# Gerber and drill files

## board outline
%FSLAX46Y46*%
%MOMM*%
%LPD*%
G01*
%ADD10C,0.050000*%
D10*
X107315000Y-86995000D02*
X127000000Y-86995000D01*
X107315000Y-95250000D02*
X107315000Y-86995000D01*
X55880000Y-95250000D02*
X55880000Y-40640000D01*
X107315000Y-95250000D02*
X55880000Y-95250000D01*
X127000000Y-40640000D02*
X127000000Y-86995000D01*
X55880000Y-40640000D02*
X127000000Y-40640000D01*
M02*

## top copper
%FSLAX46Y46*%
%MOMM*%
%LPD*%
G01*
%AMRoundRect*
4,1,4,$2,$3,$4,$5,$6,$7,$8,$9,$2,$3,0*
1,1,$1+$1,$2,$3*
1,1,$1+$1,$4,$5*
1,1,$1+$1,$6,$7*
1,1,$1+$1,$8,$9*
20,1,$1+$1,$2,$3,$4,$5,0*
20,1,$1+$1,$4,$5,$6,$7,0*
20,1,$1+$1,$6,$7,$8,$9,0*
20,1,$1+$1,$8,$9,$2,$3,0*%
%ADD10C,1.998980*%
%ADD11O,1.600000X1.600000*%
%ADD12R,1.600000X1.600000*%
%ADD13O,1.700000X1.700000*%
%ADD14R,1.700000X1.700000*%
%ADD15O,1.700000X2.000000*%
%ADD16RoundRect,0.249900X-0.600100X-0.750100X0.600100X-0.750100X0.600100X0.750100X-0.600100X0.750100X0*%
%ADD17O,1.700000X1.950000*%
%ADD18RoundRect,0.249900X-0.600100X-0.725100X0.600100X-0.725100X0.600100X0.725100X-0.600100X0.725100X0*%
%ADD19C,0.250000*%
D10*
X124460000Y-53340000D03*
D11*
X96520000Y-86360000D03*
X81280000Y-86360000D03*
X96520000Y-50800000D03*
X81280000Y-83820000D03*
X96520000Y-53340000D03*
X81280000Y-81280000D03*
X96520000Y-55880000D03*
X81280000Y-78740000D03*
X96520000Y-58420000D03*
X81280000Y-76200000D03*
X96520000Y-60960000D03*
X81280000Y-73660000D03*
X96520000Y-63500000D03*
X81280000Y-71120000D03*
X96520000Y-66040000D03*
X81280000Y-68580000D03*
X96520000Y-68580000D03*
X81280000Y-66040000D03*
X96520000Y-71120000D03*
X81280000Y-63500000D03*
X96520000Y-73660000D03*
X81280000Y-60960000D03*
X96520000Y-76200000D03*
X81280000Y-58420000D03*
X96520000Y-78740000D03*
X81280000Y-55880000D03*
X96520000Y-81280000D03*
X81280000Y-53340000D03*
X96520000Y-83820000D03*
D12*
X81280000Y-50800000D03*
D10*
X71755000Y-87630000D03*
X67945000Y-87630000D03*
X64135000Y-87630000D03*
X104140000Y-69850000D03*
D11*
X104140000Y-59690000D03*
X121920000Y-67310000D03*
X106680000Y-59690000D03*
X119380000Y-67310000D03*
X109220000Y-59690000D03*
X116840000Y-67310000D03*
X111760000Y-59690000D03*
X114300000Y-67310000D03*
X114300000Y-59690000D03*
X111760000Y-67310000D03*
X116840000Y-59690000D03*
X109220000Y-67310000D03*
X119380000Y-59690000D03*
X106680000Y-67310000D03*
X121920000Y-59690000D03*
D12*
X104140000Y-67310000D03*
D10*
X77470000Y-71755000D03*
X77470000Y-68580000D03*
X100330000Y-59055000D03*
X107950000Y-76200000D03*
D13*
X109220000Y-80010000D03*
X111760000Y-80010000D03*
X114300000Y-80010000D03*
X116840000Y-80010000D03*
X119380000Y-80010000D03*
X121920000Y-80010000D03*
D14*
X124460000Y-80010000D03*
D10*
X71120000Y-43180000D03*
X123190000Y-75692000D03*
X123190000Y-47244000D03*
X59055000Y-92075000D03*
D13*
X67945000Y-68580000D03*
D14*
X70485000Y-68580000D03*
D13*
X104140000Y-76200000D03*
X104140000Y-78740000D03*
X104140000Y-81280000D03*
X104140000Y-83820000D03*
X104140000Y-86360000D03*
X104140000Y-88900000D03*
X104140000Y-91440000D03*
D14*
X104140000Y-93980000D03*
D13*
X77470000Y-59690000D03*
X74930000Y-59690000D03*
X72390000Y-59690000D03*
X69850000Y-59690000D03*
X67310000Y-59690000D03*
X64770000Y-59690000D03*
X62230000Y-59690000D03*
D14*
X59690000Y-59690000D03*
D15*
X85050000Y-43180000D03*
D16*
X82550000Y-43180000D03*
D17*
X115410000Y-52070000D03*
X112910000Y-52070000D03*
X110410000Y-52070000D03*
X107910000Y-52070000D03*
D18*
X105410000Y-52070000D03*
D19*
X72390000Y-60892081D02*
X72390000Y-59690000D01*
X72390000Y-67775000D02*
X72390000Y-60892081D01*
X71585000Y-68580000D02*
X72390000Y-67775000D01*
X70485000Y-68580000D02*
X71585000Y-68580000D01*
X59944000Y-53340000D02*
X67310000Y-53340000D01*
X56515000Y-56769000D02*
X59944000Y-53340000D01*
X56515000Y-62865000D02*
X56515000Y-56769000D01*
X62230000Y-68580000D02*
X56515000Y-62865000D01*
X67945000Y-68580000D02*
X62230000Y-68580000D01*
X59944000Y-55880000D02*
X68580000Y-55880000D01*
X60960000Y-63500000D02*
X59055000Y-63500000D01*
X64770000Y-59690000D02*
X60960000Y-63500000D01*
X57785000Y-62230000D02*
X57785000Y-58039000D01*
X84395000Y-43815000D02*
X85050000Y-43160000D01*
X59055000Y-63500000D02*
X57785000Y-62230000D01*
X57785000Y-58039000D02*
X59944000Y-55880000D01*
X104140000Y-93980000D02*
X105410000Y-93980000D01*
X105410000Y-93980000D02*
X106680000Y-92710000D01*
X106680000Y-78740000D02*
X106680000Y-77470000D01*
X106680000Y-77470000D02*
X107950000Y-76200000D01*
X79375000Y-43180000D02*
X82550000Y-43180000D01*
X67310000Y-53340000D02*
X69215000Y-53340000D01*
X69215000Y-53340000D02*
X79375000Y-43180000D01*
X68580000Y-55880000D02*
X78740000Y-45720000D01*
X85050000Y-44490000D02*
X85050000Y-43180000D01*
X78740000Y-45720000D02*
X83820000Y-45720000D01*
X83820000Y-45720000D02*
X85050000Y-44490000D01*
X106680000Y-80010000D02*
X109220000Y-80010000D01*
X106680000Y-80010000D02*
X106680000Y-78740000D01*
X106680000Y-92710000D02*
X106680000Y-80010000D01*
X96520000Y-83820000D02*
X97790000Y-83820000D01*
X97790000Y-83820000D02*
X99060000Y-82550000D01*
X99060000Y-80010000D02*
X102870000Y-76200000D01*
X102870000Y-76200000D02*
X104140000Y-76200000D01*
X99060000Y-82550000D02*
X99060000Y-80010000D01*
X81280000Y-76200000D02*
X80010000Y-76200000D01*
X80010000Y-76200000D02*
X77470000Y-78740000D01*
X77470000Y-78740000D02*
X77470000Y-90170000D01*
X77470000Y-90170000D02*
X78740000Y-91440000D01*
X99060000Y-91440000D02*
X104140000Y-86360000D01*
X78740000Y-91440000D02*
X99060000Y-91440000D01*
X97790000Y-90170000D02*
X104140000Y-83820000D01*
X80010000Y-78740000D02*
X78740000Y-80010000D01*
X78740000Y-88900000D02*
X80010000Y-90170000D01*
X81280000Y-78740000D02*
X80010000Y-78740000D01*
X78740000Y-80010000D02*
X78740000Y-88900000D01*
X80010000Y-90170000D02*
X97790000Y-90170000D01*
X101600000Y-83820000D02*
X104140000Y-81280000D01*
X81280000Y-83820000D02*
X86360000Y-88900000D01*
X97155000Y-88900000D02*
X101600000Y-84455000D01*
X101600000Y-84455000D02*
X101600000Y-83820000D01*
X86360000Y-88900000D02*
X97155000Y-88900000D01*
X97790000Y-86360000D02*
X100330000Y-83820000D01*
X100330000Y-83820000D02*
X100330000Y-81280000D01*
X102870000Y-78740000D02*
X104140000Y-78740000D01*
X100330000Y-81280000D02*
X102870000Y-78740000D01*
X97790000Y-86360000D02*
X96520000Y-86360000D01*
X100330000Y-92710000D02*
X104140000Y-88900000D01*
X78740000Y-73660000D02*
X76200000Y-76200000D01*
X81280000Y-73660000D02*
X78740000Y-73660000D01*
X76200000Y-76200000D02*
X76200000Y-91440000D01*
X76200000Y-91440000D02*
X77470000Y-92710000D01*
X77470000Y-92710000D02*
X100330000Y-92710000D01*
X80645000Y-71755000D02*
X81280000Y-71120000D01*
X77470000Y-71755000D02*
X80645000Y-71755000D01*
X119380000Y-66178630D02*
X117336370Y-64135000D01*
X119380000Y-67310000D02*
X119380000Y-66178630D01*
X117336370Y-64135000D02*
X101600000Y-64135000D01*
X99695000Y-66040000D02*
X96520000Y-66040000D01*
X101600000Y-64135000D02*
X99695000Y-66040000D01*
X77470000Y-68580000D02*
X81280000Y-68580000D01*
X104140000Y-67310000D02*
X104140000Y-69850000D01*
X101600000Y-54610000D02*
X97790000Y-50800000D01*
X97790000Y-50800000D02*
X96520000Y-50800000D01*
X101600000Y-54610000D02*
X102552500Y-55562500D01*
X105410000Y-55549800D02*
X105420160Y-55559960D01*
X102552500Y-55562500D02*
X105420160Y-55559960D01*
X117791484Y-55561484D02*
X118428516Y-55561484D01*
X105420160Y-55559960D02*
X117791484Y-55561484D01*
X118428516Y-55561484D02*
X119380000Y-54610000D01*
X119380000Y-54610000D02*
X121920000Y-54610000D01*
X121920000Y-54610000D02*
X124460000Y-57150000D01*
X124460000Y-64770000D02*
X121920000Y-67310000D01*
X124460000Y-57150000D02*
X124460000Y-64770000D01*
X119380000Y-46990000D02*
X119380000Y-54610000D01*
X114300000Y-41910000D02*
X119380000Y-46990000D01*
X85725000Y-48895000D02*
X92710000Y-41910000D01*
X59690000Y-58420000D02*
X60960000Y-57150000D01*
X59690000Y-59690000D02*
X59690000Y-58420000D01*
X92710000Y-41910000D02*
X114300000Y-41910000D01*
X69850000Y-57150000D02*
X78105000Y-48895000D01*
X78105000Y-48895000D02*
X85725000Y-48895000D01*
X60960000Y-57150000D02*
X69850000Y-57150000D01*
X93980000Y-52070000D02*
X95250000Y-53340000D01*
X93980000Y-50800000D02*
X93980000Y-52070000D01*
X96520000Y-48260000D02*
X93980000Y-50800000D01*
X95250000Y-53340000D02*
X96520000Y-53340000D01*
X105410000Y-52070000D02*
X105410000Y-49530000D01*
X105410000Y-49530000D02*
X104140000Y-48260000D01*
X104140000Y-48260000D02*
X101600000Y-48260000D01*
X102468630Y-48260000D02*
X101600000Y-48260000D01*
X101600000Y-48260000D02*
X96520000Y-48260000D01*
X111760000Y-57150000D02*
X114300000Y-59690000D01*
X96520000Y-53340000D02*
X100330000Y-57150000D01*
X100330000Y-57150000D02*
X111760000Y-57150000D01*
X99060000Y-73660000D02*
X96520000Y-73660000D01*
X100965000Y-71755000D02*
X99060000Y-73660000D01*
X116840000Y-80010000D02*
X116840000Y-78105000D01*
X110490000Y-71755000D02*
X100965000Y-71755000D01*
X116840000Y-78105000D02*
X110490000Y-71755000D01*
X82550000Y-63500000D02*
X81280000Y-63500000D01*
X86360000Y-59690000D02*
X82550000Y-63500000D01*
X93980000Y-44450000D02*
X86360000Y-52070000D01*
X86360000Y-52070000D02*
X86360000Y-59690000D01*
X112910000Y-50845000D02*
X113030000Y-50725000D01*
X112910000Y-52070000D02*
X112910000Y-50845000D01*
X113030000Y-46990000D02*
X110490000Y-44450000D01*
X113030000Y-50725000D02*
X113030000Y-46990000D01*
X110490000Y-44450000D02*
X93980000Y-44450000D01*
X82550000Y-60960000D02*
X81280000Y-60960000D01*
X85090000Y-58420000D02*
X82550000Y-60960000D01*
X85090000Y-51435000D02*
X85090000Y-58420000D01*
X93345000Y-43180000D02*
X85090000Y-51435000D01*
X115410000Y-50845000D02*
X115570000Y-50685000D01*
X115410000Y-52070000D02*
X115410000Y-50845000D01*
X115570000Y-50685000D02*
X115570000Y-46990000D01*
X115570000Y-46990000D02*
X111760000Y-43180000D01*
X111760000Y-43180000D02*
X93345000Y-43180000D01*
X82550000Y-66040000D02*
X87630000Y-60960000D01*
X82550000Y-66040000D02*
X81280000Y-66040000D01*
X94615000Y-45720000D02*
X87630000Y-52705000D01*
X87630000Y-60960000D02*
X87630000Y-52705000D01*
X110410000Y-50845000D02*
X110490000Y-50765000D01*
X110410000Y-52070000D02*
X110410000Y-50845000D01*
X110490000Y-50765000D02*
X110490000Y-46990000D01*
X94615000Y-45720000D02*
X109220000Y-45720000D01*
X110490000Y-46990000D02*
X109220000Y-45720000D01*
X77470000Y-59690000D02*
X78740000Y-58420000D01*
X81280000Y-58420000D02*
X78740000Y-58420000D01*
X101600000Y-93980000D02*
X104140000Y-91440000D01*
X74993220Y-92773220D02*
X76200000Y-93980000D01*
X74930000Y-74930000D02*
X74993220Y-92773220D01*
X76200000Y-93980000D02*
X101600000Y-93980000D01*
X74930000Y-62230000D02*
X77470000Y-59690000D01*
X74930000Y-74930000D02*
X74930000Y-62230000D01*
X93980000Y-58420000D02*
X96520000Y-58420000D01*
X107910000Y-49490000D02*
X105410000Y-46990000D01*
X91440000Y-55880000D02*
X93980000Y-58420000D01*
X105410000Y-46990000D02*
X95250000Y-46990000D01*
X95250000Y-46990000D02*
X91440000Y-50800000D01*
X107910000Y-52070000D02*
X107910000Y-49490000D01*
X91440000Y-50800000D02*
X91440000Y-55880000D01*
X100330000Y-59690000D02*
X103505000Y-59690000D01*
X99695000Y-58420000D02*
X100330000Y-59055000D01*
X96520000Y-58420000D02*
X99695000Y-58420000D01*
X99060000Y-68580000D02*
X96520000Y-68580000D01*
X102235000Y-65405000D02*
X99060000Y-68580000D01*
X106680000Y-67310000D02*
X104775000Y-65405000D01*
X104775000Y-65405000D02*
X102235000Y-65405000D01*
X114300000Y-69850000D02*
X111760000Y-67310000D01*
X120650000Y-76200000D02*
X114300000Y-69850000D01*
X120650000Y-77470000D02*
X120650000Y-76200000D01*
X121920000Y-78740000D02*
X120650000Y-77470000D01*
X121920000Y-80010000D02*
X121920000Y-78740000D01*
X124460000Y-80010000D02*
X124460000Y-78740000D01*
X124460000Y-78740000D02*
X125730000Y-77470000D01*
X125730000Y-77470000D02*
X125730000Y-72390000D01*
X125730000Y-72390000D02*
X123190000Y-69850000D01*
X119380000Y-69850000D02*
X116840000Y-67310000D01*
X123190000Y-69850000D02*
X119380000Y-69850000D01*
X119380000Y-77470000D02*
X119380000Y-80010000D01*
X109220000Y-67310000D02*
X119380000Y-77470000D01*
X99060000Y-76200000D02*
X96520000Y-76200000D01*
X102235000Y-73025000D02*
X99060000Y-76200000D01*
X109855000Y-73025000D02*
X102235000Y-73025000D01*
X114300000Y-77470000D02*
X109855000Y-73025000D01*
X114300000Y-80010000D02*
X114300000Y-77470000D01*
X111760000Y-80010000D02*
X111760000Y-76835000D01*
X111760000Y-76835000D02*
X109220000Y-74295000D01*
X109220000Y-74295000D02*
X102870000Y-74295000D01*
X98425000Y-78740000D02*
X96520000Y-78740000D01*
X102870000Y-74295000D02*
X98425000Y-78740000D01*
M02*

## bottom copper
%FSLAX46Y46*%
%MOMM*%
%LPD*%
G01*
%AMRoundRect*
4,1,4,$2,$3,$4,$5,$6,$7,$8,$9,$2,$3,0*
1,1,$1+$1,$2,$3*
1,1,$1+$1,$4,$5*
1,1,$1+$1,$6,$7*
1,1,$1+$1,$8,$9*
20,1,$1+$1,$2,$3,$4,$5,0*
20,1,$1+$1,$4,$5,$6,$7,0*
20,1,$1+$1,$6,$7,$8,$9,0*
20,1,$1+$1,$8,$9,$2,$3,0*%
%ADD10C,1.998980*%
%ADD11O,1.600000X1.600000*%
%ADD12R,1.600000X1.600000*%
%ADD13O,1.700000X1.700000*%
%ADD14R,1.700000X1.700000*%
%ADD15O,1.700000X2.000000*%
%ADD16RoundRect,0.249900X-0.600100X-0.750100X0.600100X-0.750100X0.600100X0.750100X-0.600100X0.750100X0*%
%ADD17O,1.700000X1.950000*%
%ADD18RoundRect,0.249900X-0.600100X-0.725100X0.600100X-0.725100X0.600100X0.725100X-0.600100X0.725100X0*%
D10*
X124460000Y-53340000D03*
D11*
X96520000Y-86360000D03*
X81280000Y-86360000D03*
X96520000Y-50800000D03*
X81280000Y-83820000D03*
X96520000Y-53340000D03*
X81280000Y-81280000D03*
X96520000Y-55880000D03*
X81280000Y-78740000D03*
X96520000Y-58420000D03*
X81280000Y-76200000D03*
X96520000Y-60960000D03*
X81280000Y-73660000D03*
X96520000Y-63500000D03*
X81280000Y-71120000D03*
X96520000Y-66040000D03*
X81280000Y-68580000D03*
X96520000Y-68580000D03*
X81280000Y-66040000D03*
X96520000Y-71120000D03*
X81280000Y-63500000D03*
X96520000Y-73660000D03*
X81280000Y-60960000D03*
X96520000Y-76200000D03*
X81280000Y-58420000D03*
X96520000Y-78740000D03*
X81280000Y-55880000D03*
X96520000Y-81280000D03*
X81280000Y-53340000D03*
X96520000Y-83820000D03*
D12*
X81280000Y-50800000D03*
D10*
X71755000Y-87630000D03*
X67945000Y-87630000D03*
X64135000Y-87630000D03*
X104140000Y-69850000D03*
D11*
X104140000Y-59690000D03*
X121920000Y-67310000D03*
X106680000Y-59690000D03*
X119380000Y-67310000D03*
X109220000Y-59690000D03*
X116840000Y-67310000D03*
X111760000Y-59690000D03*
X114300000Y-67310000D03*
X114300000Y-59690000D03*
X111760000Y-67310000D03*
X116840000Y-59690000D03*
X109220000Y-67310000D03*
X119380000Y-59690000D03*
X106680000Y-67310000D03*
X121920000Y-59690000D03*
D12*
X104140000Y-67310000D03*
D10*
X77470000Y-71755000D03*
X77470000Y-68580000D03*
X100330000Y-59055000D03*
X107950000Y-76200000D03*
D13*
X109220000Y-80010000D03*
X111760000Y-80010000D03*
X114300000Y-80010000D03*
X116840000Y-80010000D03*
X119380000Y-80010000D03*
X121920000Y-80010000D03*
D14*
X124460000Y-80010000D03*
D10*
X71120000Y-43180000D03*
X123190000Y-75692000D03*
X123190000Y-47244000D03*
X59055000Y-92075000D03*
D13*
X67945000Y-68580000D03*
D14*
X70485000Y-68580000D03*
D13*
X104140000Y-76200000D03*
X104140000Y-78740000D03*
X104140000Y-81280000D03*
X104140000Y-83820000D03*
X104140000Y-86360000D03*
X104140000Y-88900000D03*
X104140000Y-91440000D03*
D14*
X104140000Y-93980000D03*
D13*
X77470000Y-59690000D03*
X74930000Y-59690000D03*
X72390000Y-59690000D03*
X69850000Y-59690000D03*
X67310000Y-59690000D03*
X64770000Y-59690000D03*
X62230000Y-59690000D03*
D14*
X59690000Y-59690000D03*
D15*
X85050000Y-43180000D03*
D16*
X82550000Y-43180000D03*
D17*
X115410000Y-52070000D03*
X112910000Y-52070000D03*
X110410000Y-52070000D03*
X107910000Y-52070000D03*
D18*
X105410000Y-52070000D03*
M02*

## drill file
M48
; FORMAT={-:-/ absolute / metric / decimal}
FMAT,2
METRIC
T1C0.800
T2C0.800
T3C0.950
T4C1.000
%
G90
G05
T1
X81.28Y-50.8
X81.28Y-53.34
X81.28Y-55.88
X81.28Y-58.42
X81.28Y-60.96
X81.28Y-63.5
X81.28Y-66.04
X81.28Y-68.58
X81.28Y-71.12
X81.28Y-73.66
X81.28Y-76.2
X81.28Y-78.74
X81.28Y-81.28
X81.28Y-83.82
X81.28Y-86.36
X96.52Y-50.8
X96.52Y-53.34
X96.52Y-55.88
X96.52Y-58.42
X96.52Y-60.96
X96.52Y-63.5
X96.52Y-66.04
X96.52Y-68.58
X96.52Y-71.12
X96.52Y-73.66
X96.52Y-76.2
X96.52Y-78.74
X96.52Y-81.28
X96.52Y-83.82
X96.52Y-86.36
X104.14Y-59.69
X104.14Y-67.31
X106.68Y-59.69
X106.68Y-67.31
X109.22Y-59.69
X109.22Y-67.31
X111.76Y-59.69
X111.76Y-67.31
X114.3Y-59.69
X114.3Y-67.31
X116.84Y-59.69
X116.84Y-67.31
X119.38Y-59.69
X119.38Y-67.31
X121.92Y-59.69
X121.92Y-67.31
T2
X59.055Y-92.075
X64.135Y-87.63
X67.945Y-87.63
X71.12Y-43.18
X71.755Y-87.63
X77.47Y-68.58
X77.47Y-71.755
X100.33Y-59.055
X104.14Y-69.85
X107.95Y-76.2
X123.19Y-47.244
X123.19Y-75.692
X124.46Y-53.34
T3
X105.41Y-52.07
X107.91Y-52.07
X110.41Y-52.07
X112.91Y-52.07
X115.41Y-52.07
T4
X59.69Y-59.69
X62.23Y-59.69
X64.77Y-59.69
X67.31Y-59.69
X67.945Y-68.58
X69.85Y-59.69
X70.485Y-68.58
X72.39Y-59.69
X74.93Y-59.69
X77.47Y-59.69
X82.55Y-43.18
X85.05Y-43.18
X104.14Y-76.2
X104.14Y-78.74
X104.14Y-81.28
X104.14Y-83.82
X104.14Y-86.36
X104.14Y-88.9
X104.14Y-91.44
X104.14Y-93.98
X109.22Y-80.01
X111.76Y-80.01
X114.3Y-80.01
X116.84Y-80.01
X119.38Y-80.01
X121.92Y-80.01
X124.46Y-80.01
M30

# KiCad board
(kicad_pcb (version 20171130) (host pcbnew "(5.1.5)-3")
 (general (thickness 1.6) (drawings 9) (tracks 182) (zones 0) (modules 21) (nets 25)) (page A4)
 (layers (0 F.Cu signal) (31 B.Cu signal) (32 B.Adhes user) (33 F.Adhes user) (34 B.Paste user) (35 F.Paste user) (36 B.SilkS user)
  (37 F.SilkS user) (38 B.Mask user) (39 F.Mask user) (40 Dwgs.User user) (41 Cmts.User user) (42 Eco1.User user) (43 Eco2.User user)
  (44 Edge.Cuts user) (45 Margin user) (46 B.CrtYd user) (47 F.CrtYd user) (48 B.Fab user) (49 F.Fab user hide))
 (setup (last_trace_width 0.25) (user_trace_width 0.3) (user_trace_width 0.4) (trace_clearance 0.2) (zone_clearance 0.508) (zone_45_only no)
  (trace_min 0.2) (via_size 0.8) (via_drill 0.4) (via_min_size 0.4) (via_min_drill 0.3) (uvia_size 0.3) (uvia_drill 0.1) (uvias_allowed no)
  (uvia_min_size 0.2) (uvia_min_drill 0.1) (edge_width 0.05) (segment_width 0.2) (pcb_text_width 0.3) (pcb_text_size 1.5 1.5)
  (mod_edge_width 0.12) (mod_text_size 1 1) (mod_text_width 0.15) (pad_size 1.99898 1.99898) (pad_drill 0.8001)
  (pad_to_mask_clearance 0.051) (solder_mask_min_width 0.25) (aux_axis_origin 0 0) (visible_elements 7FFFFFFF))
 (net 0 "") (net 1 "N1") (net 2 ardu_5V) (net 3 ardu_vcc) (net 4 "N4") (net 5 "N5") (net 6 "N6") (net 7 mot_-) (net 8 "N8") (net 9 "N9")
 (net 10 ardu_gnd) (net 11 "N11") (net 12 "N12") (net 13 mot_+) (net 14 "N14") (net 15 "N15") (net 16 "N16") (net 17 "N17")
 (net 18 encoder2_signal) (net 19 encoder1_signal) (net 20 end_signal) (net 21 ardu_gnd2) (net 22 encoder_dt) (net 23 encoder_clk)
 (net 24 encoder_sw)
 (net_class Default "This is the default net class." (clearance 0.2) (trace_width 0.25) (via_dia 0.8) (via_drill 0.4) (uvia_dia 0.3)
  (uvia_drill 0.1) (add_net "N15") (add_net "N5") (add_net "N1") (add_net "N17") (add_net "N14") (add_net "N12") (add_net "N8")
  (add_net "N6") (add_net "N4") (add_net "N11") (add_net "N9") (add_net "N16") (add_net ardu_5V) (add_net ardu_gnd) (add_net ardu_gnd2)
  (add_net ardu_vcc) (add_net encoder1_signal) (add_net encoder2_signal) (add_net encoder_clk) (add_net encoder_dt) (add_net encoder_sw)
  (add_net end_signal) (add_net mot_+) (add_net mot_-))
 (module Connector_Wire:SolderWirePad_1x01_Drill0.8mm (layer F.Cu) (at 124.46 53.34)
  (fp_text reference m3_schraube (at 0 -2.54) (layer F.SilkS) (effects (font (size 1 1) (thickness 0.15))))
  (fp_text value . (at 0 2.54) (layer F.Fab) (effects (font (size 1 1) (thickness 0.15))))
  (pad 1 thru_hole circle (at 0 0) (size 1.99898 1.99898) (drill 0.8001) (layers *.Cu *.Mask)))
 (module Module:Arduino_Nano (layer F.Cu) (at 81.28 50.8)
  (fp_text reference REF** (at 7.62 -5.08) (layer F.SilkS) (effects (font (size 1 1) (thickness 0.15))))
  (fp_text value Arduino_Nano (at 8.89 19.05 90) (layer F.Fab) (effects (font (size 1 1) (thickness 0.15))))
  (pad 16 thru_hole oval (at 15.24 35.56) (size 1.6 1.6) (drill 0.8) (layers *.Cu *.Mask))
  (pad 15 thru_hole oval (at 0 35.56) (size 1.6 1.6) (drill 0.8) (layers *.Cu *.Mask))
  (pad 30 thru_hole oval (at 15.24 0) (size 1.6 1.6) (drill 0.8) (layers *.Cu *.Mask))
  (pad 14 thru_hole oval (at 0 33.02) (size 1.6 1.6) (drill 0.8) (layers *.Cu *.Mask))
  (pad 29 thru_hole oval (at 15.24 2.54) (size 1.6 1.6) (drill 0.8) (layers *.Cu *.Mask))
  (pad 13 thru_hole oval (at 0 30.48) (size 1.6 1.6) (drill 0.8) (layers *.Cu *.Mask))
  (pad 28 thru_hole oval (at 15.24 5.08) (size 1.6 1.6) (drill 0.8) (layers *.Cu *.Mask))
  (pad 12 thru_hole oval (at 0 27.94) (size 1.6 1.6) (drill 0.8) (layers *.Cu *.Mask))
  (pad 27 thru_hole oval (at 15.24 7.62) (size 1.6 1.6) (drill 0.8) (layers *.Cu *.Mask))
  (pad 11 thru_hole oval (at 0 25.4) (size 1.6 1.6) (drill 0.8) (layers *.Cu *.Mask))
  (pad 26 thru_hole oval (at 15.24 10.16) (size 1.6 1.6) (drill 0.8) (layers *.Cu *.Mask))
  (pad 10 thru_hole oval (at 0 22.86) (size 1.6 1.6) (drill 0.8) (layers *.Cu *.Mask))
  (pad 25 thru_hole oval (at 15.24 12.7) (size 1.6 1.6) (drill 0.8) (layers *.Cu *.Mask))
  (pad 9 thru_hole oval (at 0 20.32) (size 1.6 1.6) (drill 0.8) (layers *.Cu *.Mask))
  (pad 24 thru_hole oval (at 15.24 15.24) (size 1.6 1.6) (drill 0.8) (layers *.Cu *.Mask))
  (pad 8 thru_hole oval (at 0 17.78) (size 1.6 1.6) (drill 0.8) (layers *.Cu *.Mask))
  (pad 23 thru_hole oval (at 15.24 17.78) (size 1.6 1.6) (drill 0.8) (layers *.Cu *.Mask))
  (pad 7 thru_hole oval (at 0 15.24) (size 1.6 1.6) (drill 0.8) (layers *.Cu *.Mask))
  (pad 22 thru_hole oval (at 15.24 20.32) (size 1.6 1.6) (drill 0.8) (layers *.Cu *.Mask))
  (pad 6 thru_hole oval (at 0 12.7) (size 1.6 1.6) (drill 0.8) (layers *.Cu *.Mask))
  (pad 21 thru_hole oval (at 15.24 22.86) (size 1.6 1.6) (drill 0.8) (layers *.Cu *.Mask))
  (pad 5 thru_hole oval (at 0 10.16) (size 1.6 1.6) (drill 0.8) (layers *.Cu *.Mask))
  (pad 20 thru_hole oval (at 15.24 25.4) (size 1.6 1.6) (drill 0.8) (layers *.Cu *.Mask))
  (pad 4 thru_hole oval (at 0 7.62) (size 1.6 1.6) (drill 0.8) (layers *.Cu *.Mask))
  (pad 19 thru_hole oval (at 15.24 27.94) (size 1.6 1.6) (drill 0.8) (layers *.Cu *.Mask))
  (pad 3 thru_hole oval (at 0 5.08) (size 1.6 1.6) (drill 0.8) (layers *.Cu *.Mask))
  (pad 18 thru_hole oval (at 15.24 30.48) (size 1.6 1.6) (drill 0.8) (layers *.Cu *.Mask))
  (pad 2 thru_hole oval (at 0 2.54) (size 1.6 1.6) (drill 0.8) (layers *.Cu *.Mask))
  (pad 17 thru_hole oval (at 15.24 33.02) (size 1.6 1.6) (drill 0.8) (layers *.Cu *.Mask))
  (pad 1 thru_hole rect (at 0 0) (size 1.6 1.6) (drill 0.8) (layers *.Cu *.Mask)))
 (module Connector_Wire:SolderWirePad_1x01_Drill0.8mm (layer F.Cu) (at 71.755 87.63)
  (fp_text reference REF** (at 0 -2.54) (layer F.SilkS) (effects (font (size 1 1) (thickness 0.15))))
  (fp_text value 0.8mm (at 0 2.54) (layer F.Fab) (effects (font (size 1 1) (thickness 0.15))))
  (pad 1 thru_hole circle (at 0 0) (size 1.99898 1.99898) (drill 0.8001) (layers *.Cu *.Mask)))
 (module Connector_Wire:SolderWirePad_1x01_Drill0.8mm (layer F.Cu) (at 67.945 87.63)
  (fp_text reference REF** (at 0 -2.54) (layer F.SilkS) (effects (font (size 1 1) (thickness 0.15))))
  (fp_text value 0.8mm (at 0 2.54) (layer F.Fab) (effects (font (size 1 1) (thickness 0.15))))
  (pad 1 thru_hole circle (at 0 0) (size 1.99898 1.99898) (drill 0.8001) (layers *.Cu *.Mask)))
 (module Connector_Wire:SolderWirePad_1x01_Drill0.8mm (layer F.Cu) (at 64.135 87.63)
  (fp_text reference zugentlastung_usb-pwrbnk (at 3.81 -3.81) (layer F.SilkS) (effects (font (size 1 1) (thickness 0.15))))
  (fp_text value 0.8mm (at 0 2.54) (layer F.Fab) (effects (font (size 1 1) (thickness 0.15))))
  (pad 1 thru_hole circle (at 0 0) (size 1.99898 1.99898) (drill 0.8001) (layers *.Cu *.Mask)))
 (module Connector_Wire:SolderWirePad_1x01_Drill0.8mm (layer F.Cu) (at 104.14 69.85)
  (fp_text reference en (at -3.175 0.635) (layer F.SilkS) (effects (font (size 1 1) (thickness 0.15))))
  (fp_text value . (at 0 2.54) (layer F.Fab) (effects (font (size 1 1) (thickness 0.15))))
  (pad 1 thru_hole circle (at 0 0) (size 1.99898 1.99898) (drill 0.8001) (layers *.Cu *.Mask) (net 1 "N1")))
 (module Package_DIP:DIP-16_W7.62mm (layer F.Cu) (at 104.14 67.31 90)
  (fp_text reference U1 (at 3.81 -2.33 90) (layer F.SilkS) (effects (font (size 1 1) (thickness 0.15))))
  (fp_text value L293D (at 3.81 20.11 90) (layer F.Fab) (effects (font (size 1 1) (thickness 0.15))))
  (pad 16 thru_hole oval (at 7.62 0 90) (size 1.6 1.6) (drill 0.8) (layers *.Cu *.Mask) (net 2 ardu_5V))
  (pad 8 thru_hole oval (at 0 17.78 90) (size 1.6 1.6) (drill 0.8) (layers *.Cu *.Mask) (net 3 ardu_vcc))
  (pad 15 thru_hole oval (at 7.62 2.54 90) (size 1.6 1.6) (drill 0.8) (layers *.Cu *.Mask) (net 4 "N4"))
  (pad 7 thru_hole oval (at 0 15.24 90) (size 1.6 1.6) (drill 0.8) (layers *.Cu *.Mask) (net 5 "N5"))
  (pad 14 thru_hole oval (at 7.62 5.08 90) (size 1.6 1.6) (drill 0.8) (layers *.Cu *.Mask) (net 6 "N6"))
  (pad 6 thru_hole oval (at 0 12.7 90) (size 1.6 1.6) (drill 0.8) (layers *.Cu *.Mask) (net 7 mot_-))
  (pad 13 thru_hole oval (at 7.62 7.62 90) (size 1.6 1.6) (drill 0.8) (layers *.Cu *.Mask) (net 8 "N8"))
  (pad 5 thru_hole oval (at 0 10.16 90) (size 1.6 1.6) (drill 0.8) (layers *.Cu *.Mask) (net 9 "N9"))
  (pad 12 thru_hole oval (at 7.62 10.16 90) (size 1.6 1.6) (drill 0.8) (layers *.Cu *.Mask) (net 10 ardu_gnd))
  (pad 4 thru_hole oval (at 0 7.62 90) (size 1.6 1.6) (drill 0.8) (layers *.Cu *.Mask) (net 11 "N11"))
  (pad 11 thru_hole oval (at 7.62 12.7 90) (size 1.6 1.6) (drill 0.8) (layers *.Cu *.Mask) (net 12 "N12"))
  (pad 3 thru_hole oval (at 0 5.08 90) (size 1.6 1.6) (drill 0.8) (layers *.Cu *.Mask) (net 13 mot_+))
  (pad 10 thru_hole oval (at 7.62 15.24 90) (size 1.6 1.6) (drill 0.8) (layers *.Cu *.Mask) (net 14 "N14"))
  (pad 2 thru_hole oval (at 0 2.54 90) (size 1.6 1.6) (drill 0.8) (layers *.Cu *.Mask) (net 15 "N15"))
  (pad 9 thru_hole oval (at 7.62 17.78 90) (size 1.6 1.6) (drill 0.8) (layers *.Cu *.Mask) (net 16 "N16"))
  (pad 1 thru_hole rect (at 0 0 90) (size 1.6 1.6) (drill 0.8) (layers *.Cu *.Mask) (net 1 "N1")))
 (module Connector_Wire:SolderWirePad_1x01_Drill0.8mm (layer F.Cu) (at 77.47 71.755)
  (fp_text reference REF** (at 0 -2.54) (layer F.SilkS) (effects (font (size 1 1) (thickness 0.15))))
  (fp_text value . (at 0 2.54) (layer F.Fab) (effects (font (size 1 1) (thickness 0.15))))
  (pad 1 thru_hole circle (at 0 0) (size 1.99898 1.99898) (drill 0.8001) (layers *.Cu *.Mask) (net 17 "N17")))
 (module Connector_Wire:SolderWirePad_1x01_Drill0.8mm (layer F.Cu) (at 77.47 68.58)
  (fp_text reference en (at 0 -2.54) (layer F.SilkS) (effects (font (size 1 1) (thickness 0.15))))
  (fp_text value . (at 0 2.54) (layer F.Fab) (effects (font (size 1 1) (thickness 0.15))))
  (pad 1 thru_hole circle (at 0 0) (size 1.99898 1.99898) (drill 0.8001) (layers *.Cu *.Mask) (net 1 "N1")))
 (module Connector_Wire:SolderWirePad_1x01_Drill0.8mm (layer F.Cu) (at 100.33 59.055)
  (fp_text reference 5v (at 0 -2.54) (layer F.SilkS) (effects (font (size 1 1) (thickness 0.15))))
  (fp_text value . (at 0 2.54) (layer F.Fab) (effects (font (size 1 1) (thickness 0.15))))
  (pad 1 thru_hole circle (at 0 0) (size 1.99898 1.99898) (drill 0.8001) (layers *.Cu *.Mask) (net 2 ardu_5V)))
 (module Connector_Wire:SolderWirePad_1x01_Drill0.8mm (layer F.Cu) (at 107.95 76.2)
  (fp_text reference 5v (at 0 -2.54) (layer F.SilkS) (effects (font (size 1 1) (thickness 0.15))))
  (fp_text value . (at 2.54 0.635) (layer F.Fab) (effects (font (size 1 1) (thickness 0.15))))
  (pad 1 thru_hole circle (at 0 0) (size 1.99898 1.99898) (drill 0.8001) (layers *.Cu *.Mask)))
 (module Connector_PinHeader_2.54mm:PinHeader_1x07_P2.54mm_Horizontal (layer F.Cu) (at 124.46 80.01 270)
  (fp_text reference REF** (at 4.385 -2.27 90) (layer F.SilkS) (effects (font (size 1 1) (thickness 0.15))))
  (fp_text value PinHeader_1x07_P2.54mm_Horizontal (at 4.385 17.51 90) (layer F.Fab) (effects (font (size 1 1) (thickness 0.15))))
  (pad 7 thru_hole oval (at 0 15.24 270) (size 1.7 1.7) (drill 1) (layers *.Cu *.Mask))
  (pad 6 thru_hole oval (at 0 12.7 270) (size 1.7 1.7) (drill 1) (layers *.Cu *.Mask) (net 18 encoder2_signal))
  (pad 5 thru_hole oval (at 0 10.16 270) (size 1.7 1.7) (drill 1) (layers *.Cu *.Mask) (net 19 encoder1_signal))
  (pad 4 thru_hole oval (at 0 7.62 270) (size 1.7 1.7) (drill 1) (layers *.Cu *.Mask) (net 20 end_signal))
  (pad 3 thru_hole oval (at 0 5.08 270) (size 1.7 1.7) (drill 1) (layers *.Cu *.Mask) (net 13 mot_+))
  (pad 2 thru_hole oval (at 0 2.54 270) (size 1.7 1.7) (drill 1) (layers *.Cu *.Mask) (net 11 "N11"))
  (pad 1 thru_hole rect (at 0 0 270) (size 1.7 1.7) (drill 1) (layers *.Cu *.Mask) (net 7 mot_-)))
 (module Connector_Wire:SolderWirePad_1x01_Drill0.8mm (layer F.Cu) (at 71.12 43.18)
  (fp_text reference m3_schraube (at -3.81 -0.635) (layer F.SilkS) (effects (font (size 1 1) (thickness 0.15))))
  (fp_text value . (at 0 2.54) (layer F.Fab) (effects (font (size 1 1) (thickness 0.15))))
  (pad 1 thru_hole circle (at 0 0) (size 1.99898 1.99898) (drill 0.8001) (layers *.Cu *.Mask)))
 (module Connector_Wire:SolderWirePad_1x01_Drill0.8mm (layer F.Cu) (at 123.19 75.692)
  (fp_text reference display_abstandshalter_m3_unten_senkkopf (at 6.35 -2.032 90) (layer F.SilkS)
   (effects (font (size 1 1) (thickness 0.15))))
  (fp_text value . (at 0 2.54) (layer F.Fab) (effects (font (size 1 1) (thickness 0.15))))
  (pad 1 thru_hole circle (at 0 0) (size 1.99898 1.99898) (drill 0.8001) (layers *.Cu *.Mask)))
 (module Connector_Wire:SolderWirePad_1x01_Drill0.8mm (layer F.Cu) (at 123.19 47.244)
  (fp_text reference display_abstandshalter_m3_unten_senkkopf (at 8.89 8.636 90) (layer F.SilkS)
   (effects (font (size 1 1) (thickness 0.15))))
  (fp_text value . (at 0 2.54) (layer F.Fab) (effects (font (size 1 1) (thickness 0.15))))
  (pad 1 thru_hole circle (at 0 0) (size 1.99898 1.99898) (drill 0.8001) (layers *.Cu *.Mask)))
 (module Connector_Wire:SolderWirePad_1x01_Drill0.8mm (layer F.Cu) (at 59.055 92.075)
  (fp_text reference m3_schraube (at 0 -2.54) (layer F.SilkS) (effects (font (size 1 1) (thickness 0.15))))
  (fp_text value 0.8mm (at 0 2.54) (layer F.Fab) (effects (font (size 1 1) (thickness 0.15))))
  (pad 1 thru_hole circle (at 0 0) (size 1.99898 1.99898) (drill 0.8001) (layers *.Cu *.Mask)))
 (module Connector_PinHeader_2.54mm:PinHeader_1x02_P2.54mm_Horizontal (layer F.Cu) (at 70.485 68.58 270)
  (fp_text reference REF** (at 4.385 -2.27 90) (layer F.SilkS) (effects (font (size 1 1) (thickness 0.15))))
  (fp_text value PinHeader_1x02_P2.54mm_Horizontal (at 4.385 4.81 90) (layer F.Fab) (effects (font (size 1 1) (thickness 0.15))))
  (pad 2 thru_hole oval (at 0 2.54 270) (size 1.7 1.7) (drill 1) (layers *.Cu *.Mask))
  (pad 1 thru_hole rect (at 0 0 270) (size 1.7 1.7) (drill 1) (layers *.Cu *.Mask)))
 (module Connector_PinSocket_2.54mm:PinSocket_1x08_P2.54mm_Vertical (layer F.Cu) (at 104.14 93.98 180)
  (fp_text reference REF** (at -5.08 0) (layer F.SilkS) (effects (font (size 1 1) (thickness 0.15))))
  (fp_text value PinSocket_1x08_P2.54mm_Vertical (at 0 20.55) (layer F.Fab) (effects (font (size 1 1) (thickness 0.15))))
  (pad 8 thru_hole oval (at 0 17.78 180) (size 1.7 1.7) (drill 1) (layers *.Cu *.Mask))
  (pad 7 thru_hole oval (at 0 15.24 180) (size 1.7 1.7) (drill 1) (layers *.Cu *.Mask))
  (pad 6 thru_hole oval (at 0 12.7 180) (size 1.7 1.7) (drill 1) (layers *.Cu *.Mask))
  (pad 5 thru_hole oval (at 0 10.16 180) (size 1.7 1.7) (drill 1) (layers *.Cu *.Mask))
  (pad 4 thru_hole oval (at 0 7.62 180) (size 1.7 1.7) (drill 1) (layers *.Cu *.Mask))
  (pad 3 thru_hole oval (at 0 5.08 180) (size 1.7 1.7) (drill 1) (layers *.Cu *.Mask))
  (pad 2 thru_hole oval (at 0 2.54 180) (size 1.7 1.7) (drill 1) (layers *.Cu *.Mask))
  (pad 1 thru_hole rect (at 0 0 180) (size 1.7 1.7) (drill 1) (layers *.Cu *.Mask)))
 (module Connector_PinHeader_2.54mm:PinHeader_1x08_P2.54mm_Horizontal (layer F.Cu) (at 59.69 59.69 90)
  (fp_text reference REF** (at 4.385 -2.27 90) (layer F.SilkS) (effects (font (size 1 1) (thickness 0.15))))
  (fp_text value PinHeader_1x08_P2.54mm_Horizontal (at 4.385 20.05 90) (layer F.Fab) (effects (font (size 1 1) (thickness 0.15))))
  (pad 8 thru_hole oval (at 0 17.78 90) (size 1.7 1.7) (drill 1) (layers *.Cu *.Mask) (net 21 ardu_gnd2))
  (pad 7 thru_hole oval (at 0 15.24 90) (size 1.7 1.7) (drill 1) (layers *.Cu *.Mask))
  (pad 6 thru_hole oval (at 0 12.7 90) (size 1.7 1.7) (drill 1) (layers *.Cu *.Mask))
  (pad 5 thru_hole oval (at 0 10.16 90) (size 1.7 1.7) (drill 1) (layers *.Cu *.Mask))
  (pad 4 thru_hole oval (at 0 7.62 90) (size 1.7 1.7) (drill 1) (layers *.Cu *.Mask))
  (pad 3 thru_hole oval (at 0 5.08 90) (size 1.7 1.7) (drill 1) (layers *.Cu *.Mask))
  (pad 2 thru_hole oval (at 0 2.54 90) (size 1.7 1.7) (drill 1) (layers *.Cu *.Mask))
  (pad 1 thru_hole rect (at 0 0 90) (size 1.7 1.7) (drill 1) (layers *.Cu *.Mask) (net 3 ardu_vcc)))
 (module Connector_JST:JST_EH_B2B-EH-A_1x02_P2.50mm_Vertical (layer F.Cu) (at 82.55 43.18)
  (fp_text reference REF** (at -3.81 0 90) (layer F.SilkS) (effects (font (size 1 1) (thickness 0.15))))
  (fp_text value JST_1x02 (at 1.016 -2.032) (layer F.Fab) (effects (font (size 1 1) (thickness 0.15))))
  (pad 2 thru_hole oval (at 2.5 0) (size 1.7 2) (drill 1) (layers *.Cu *.Mask))
  (pad 1 thru_hole roundrect (at 0 0) (size 1.7 2) (drill 1) (layers *.Cu *.Mask) (roundrect_rratio 0.147)))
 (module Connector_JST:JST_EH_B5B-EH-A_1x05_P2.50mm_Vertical (layer F.Cu) (at 105.41 52.07)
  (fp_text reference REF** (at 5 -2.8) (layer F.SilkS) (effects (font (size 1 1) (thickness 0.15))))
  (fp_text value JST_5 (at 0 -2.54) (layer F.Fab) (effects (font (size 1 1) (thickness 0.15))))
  (pad 5 thru_hole oval (at 10 0) (size 1.7 1.95) (drill 0.95) (layers *.Cu *.Mask) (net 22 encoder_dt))
  (pad 4 thru_hole oval (at 7.5 0) (size 1.7 1.95) (drill 0.95) (layers *.Cu *.Mask) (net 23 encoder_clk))
  (pad 3 thru_hole oval (at 5 0) (size 1.7 1.95) (drill 0.95) (layers *.Cu *.Mask) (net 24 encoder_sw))
  (pad 2 thru_hole oval (at 2.5 0) (size 1.7 1.95) (drill 0.95) (layers *.Cu *.Mask) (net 2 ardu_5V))
  (pad 1 thru_hole roundrect (at 0 0) (size 1.7 1.95) (drill 0.95) (layers *.Cu *.Mask) (roundrect_rratio 0.147) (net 10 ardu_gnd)))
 (gr_line (start 107.315 86.995) (end 127 86.995) (layer Edge.Cuts) (width 0.05))
 (gr_line (start 107.315 95.25) (end 107.315 86.995) (layer Edge.Cuts) (width 0.05))
 (gr_line (start 55.88 95.25) (end 55.88 40.64) (layer Edge.Cuts) (width 0.05))
 (gr_line (start 107.315 95.25) (end 55.88 95.25) (layer Edge.Cuts) (width 0.05))
 (gr_line (start 127 40.64) (end 127 86.995) (layer Edge.Cuts) (width 0.05))
 (gr_line (start 55.88 40.64) (end 127 40.64) (layer Edge.Cuts) (width 0.05))
 (segment (start 72.39 60.892081) (end 72.39 59.69) (width 0.25) (layer F.Cu) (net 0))
 (segment (start 72.39 67.775) (end 72.39 60.892081) (width 0.25) (layer F.Cu) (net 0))
 (segment (start 71.585 68.58) (end 72.39 67.775) (width 0.25) (layer F.Cu) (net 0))
 (segment (start 70.485 68.58) (end 71.585 68.58) (width 0.25) (layer F.Cu) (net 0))
 (segment (start 59.944 53.34) (end 67.31 53.34) (width 0.25) (layer F.Cu) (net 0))
 (segment (start 56.515 56.769) (end 59.944 53.34) (width 0.25) (layer F.Cu) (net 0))
 (segment (start 56.515 62.865) (end 56.515 56.769) (width 0.25) (layer F.Cu) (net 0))
 (segment (start 62.23 68.58) (end 56.515 62.865) (width 0.25) (layer F.Cu) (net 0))
 (segment (start 67.945 68.58) (end 62.23 68.58) (width 0.25) (layer F.Cu) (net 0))
 (segment (start 59.944 55.88) (end 68.58 55.88) (width 0.25) (layer F.Cu) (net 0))
 (segment (start 60.96 63.5) (end 59.055 63.5) (width 0.25) (layer F.Cu) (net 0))
 (segment (start 64.77 59.69) (end 60.96 63.5) (width 0.25) (layer F.Cu) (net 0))
 (segment (start 57.785 62.23) (end 57.785 58.039) (width 0.25) (layer F.Cu) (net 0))
 (segment (start 84.395 43.815) (end 85.05 43.16) (width 0.25) (layer F.Cu) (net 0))
 (segment (start 59.055 63.5) (end 57.785 62.23) (width 0.25) (layer F.Cu) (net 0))
 (segment (start 57.785 58.039) (end 59.944 55.88) (width 0.25) (layer F.Cu) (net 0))
 (segment (start 104.14 93.98) (end 105.41 93.98) (width 0.25) (layer F.Cu) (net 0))
 (segment (start 105.41 93.98) (end 106.68 92.71) (width 0.25) (layer F.Cu) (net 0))
 (segment (start 106.68 78.74) (end 106.68 77.47) (width 0.25) (layer F.Cu) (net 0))
 (segment (start 106.68 77.47) (end 107.95 76.2) (width 0.25) (layer F.Cu) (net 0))
 (segment (start 79.375 43.18) (end 82.55 43.18) (width 0.25) (layer F.Cu) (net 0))
 (segment (start 67.31 53.34) (end 69.215 53.34) (width 0.25) (layer F.Cu) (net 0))
 (segment (start 69.215 53.34) (end 79.375 43.18) (width 0.25) (layer F.Cu) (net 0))
 (segment (start 68.58 55.88) (end 78.74 45.72) (width 0.25) (layer F.Cu) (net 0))
 (segment (start 85.05 44.49) (end 85.05 43.18) (width 0.25) (layer F.Cu) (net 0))
 (segment (start 78.74 45.72) (end 83.82 45.72) (width 0.25) (layer F.Cu) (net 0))
 (segment (start 83.82 45.72) (end 85.05 44.49) (width 0.25) (layer F.Cu) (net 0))
 (segment (start 106.68 80.01) (end 109.22 80.01) (width 0.25) (layer F.Cu) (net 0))
 (segment (start 106.68 80.01) (end 106.68 78.74) (width 0.25) (layer F.Cu) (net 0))
 (segment (start 106.68 92.71) (end 106.68 80.01) (width 0.25) (layer F.Cu) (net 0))
 (segment (start 96.52 83.82) (end 97.79 83.82) (width 0.25) (layer F.Cu) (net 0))
 (segment (start 97.79 83.82) (end 99.06 82.55) (width 0.25) (layer F.Cu) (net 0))
 (segment (start 99.06 80.01) (end 102.87 76.2) (width 0.25) (layer F.Cu) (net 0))
 (segment (start 102.87 76.2) (end 104.14 76.2) (width 0.25) (layer F.Cu) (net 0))
 (segment (start 99.06 82.55) (end 99.06 80.01) (width 0.25) (layer F.Cu) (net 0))
 (segment (start 81.28 76.2) (end 80.01 76.2) (width 0.25) (layer F.Cu) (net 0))
 (segment (start 80.01 76.2) (end 77.47 78.74) (width 0.25) (layer F.Cu) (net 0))
 (segment (start 77.47 78.74) (end 77.47 90.17) (width 0.25) (layer F.Cu) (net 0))
 (segment (start 77.47 90.17) (end 78.74 91.44) (width 0.25) (layer F.Cu) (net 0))
 (segment (start 99.06 91.44) (end 104.14 86.36) (width 0.25) (layer F.Cu) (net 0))
 (segment (start 78.74 91.44) (end 99.06 91.44) (width 0.25) (layer F.Cu) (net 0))
 (segment (start 97.79 90.17) (end 104.14 83.82) (width 0.25) (layer F.Cu) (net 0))
 (segment (start 80.01 78.74) (end 78.74 80.01) (width 0.25) (layer F.Cu) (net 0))
 (segment (start 78.74 88.9) (end 80.01 90.17) (width 0.25) (layer F.Cu) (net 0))
 (segment (start 81.28 78.74) (end 80.01 78.74) (width 0.25) (layer F.Cu) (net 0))
 (segment (start 78.74 80.01) (end 78.74 88.9) (width 0.25) (layer F.Cu) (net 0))
 (segment (start 80.01 90.17) (end 97.79 90.17) (width 0.25) (layer F.Cu) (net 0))
 (segment (start 101.6 83.82) (end 104.14 81.28) (width 0.25) (layer F.Cu) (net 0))
 (segment (start 81.28 83.82) (end 86.36 88.9) (width 0.25) (layer F.Cu) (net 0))
 (segment (start 97.155 88.9) (end 101.6 84.455) (width 0.25) (layer F.Cu) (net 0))
 (segment (start 101.6 84.455) (end 101.6 83.82) (width 0.25) (layer F.Cu) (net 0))
 (segment (start 86.36 88.9) (end 97.155 88.9) (width 0.25) (layer F.Cu) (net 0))
 (segment (start 97.79 86.36) (end 100.33 83.82) (width 0.25) (layer F.Cu) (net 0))
 (segment (start 100.33 83.82) (end 100.33 81.28) (width 0.25) (layer F.Cu) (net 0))
 (segment (start 102.87 78.74) (end 104.14 78.74) (width 0.25) (layer F.Cu) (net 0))
 (segment (start 100.33 81.28) (end 102.87 78.74) (width 0.25) (layer F.Cu) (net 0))
 (segment (start 97.79 86.36) (end 96.52 86.36) (width 0.25) (layer F.Cu) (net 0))
 (segment (start 100.33 92.71) (end 104.14 88.9) (width 0.25) (layer F.Cu) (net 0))
 (segment (start 78.74 73.66) (end 76.2 76.2) (width 0.25) (layer F.Cu) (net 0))
 (segment (start 81.28 73.66) (end 78.74 73.66) (width 0.25) (layer F.Cu) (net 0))
 (segment (start 76.2 76.2) (end 76.2 91.44) (width 0.25) (layer F.Cu) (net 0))
 (segment (start 76.2 91.44) (end 77.47 92.71) (width 0.25) (layer F.Cu) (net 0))
 (segment (start 77.47 92.71) (end 100.33 92.71) (width 0.25) (layer F.Cu) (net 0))
 (segment (start 80.645 71.755) (end 81.28 71.12) (width 0.25) (layer F.Cu) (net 17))
 (segment (start 77.47 71.755) (end 80.645 71.755) (width 0.25) (layer F.Cu) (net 17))
 (segment (start 119.38 66.17863) (end 117.33637 64.135) (width 0.25) (layer F.Cu) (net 5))
 (segment (start 119.38 67.31) (end 119.38 66.17863) (width 0.25) (layer F.Cu) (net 5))
 (segment (start 117.33637 64.135) (end 101.6 64.135) (width 0.25) (layer F.Cu) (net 5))
 (segment (start 99.695 66.04) (end 96.52 66.04) (width 0.25) (layer F.Cu) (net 5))
 (segment (start 101.6 64.135) (end 99.695 66.04) (width 0.25) (layer F.Cu) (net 5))
 (segment (start 77.47 68.58) (end 81.28 68.58) (width 0.25) (layer F.Cu) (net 1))
 (segment (start 104.14 67.31) (end 104.14 69.85) (width 0.25) (layer F.Cu) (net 1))
 (segment (start 101.6 54.61) (end 97.79 50.8) (width 0.25) (layer F.Cu) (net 3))
 (segment (start 97.79 50.8) (end 96.52 50.8) (width 0.25) (layer F.Cu) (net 3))
 (segment (start 101.6 54.61) (end 102.5525 55.5625) (width 0.25) (layer F.Cu) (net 3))
 (segment (start 105.41 55.5498) (end 105.42016 55.55996) (width 0.25) (layer F.Cu) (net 3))
 (segment (start 102.5525 55.5625) (end 105.42016 55.55996) (width 0.25) (layer F.Cu) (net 3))
 (segment (start 117.791484 55.561484) (end 118.428516 55.561484) (width 0.25) (layer F.Cu) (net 3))
 (segment (start 105.42016 55.55996) (end 117.791484 55.561484) (width 0.25) (layer F.Cu) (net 3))
 (segment (start 118.428516 55.561484) (end 119.38 54.61) (width 0.25) (layer F.Cu) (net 3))
 (segment (start 119.38 54.61) (end 121.92 54.61) (width 0.25) (layer F.Cu) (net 3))
 (segment (start 121.92 54.61) (end 124.46 57.15) (width 0.25) (layer F.Cu) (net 3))
 (segment (start 124.46 64.77) (end 121.92 67.31) (width 0.25) (layer F.Cu) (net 3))
 (segment (start 124.46 57.15) (end 124.46 64.77) (width 0.25) (layer F.Cu) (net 3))
 (segment (start 119.38 46.99) (end 119.38 54.61) (width 0.25) (layer F.Cu) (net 3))
 (segment (start 114.3 41.91) (end 119.38 46.99) (width 0.25) (layer F.Cu) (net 3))
 (segment (start 85.725 48.895) (end 92.71 41.91) (width 0.25) (layer F.Cu) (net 3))
 (segment (start 59.69 58.42) (end 60.96 57.15) (width 0.25) (layer F.Cu) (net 3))
 (segment (start 59.69 59.69) (end 59.69 58.42) (width 0.25) (layer F.Cu) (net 3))
 (segment (start 92.71 41.91) (end 114.3 41.91) (width 0.25) (layer F.Cu) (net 3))
 (segment (start 69.85 57.15) (end 78.105 48.895) (width 0.25) (layer F.Cu) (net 3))
 (segment (start 78.105 48.895) (end 85.725 48.895) (width 0.25) (layer F.Cu) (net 3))
 (segment (start 60.96 57.15) (end 69.85 57.15) (width 0.25) (layer F.Cu) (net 3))
 (segment (start 93.98 52.07) (end 95.25 53.34) (width 0.25) (layer F.Cu) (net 10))
 (segment (start 93.98 50.8) (end 93.98 52.07) (width 0.25) (layer F.Cu) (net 10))
 (segment (start 96.52 48.26) (end 93.98 50.8) (width 0.25) (layer F.Cu) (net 10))
 (segment (start 95.25 53.34) (end 96.52 53.34) (width 0.25) (layer F.Cu) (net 10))
 (segment (start 105.41 52.07) (end 105.41 49.53) (width 0.25) (layer F.Cu) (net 10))
 (segment (start 105.41 49.53) (end 104.14 48.26) (width 0.25) (layer F.Cu) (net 10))
 (segment (start 104.14 48.26) (end 101.6 48.26) (width 0.25) (layer F.Cu) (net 10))
 (segment (start 102.46863 48.26) (end 101.6 48.26) (width 0.25) (layer F.Cu) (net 10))
 (segment (start 101.6 48.26) (end 96.52 48.26) (width 0.25) (layer F.Cu) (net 10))
 (segment (start 111.76 57.15) (end 114.3 59.69) (width 0.25) (layer F.Cu) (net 10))
 (segment (start 96.52 53.34) (end 100.33 57.15) (width 0.25) (layer F.Cu) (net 10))
 (segment (start 100.33 57.15) (end 111.76 57.15) (width 0.25) (layer F.Cu) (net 10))
 (segment (start 99.06 73.66) (end 96.52 73.66) (width 0.25) (layer F.Cu) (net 20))
 (segment (start 100.965 71.755) (end 99.06 73.66) (width 0.25) (layer F.Cu) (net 20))
 (segment (start 116.84 80.01) (end 116.84 78.105) (width 0.25) (layer F.Cu) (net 20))
 (segment (start 110.49 71.755) (end 100.965 71.755) (width 0.25) (layer F.Cu) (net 20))
 (segment (start 116.84 78.105) (end 110.49 71.755) (width 0.25) (layer F.Cu) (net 20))
 (segment (start 82.55 63.5) (end 81.28 63.5) (width 0.25) (layer F.Cu) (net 23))
 (segment (start 86.36 59.69) (end 82.55 63.5) (width 0.25) (layer F.Cu) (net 23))
 (segment (start 93.98 44.45) (end 86.36 52.07) (width 0.25) (layer F.Cu) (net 23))
 (segment (start 86.36 52.07) (end 86.36 59.69) (width 0.25) (layer F.Cu) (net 23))
 (segment (start 112.91 50.845) (end 113.03 50.725) (width 0.25) (layer F.Cu) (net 23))
 (segment (start 112.91 52.07) (end 112.91 50.845) (width 0.25) (layer F.Cu) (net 23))
 (segment (start 113.03 46.99) (end 110.49 44.45) (width 0.25) (layer F.Cu) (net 23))
 (segment (start 113.03 50.725) (end 113.03 46.99) (width 0.25) (layer F.Cu) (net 23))
 (segment (start 110.49 44.45) (end 93.98 44.45) (width 0.25) (layer F.Cu) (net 23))
 (segment (start 82.55 60.96) (end 81.28 60.96) (width 0.25) (layer F.Cu) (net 22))
 (segment (start 85.09 58.42) (end 82.55 60.96) (width 0.25) (layer F.Cu) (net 22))
 (segment (start 85.09 51.435) (end 85.09 58.42) (width 0.25) (layer F.Cu) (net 22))
 (segment (start 93.345 43.18) (end 85.09 51.435) (width 0.25) (layer F.Cu) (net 22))
 (segment (start 115.41 50.845) (end 115.57 50.685) (width 0.25) (layer F.Cu) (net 22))
 (segment (start 115.41 52.07) (end 115.41 50.845) (width 0.25) (layer F.Cu) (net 22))
 (segment (start 115.57 50.685) (end 115.57 46.99) (width 0.25) (layer F.Cu) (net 22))
 (segment (start 115.57 46.99) (end 111.76 43.18) (width 0.25) (layer F.Cu) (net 22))
 (segment (start 111.76 43.18) (end 93.345 43.18) (width 0.25) (layer F.Cu) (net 22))
 (segment (start 82.55 66.04) (end 87.63 60.96) (width 0.25) (layer F.Cu) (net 24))
 (segment (start 82.55 66.04) (end 81.28 66.04) (width 0.25) (layer F.Cu) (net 24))
 (segment (start 94.615 45.72) (end 87.63 52.705) (width 0.25) (layer F.Cu) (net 24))
 (segment (start 87.63 60.96) (end 87.63 52.705) (width 0.25) (layer F.Cu) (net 24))
 (segment (start 110.41 50.845) (end 110.49 50.765) (width 0.25) (layer F.Cu) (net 24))
 (segment (start 110.41 52.07) (end 110.41 50.845) (width 0.25) (layer F.Cu) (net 24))
 (segment (start 110.49 50.765) (end 110.49 46.99) (width 0.25) (layer F.Cu) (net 24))
 (segment (start 94.615 45.72) (end 109.22 45.72) (width 0.25) (layer F.Cu) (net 24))
 (segment (start 110.49 46.99) (end 109.22 45.72) (width 0.25) (layer F.Cu) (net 24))
 (segment (start 77.47 59.69) (end 78.74 58.42) (width 0.25) (layer F.Cu) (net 21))
 (segment (start 81.28 58.42) (end 78.74 58.42) (width 0.25) (layer F.Cu) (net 21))
 (segment (start 101.6 93.98) (end 104.14 91.44) (width 0.25) (layer F.Cu) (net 21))
 (segment (start 74.99322 92.77322) (end 76.2 93.98) (width 0.25) (layer F.Cu) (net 21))
 (segment (start 74.93 74.93) (end 74.99322 92.77322) (width 0.25) (layer F.Cu) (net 21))
 (segment (start 76.2 93.98) (end 101.6 93.98) (width 0.25) (layer F.Cu) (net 21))
 (segment (start 74.93 62.23) (end 77.47 59.69) (width 0.25) (layer F.Cu) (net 21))
 (segment (start 74.93 74.93) (end 74.93 62.23) (width 0.25) (layer F.Cu) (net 21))
 (segment (start 93.98 58.42) (end 96.52 58.42) (width 0.25) (layer F.Cu) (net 2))
 (segment (start 107.91 49.49) (end 105.41 46.99) (width 0.25) (layer F.Cu) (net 2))
 (segment (start 91.44 55.88) (end 93.98 58.42) (width 0.25) (layer F.Cu) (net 2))
 (segment (start 105.41 46.99) (end 95.25 46.99) (width 0.25) (layer F.Cu) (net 2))
 (segment (start 95.25 46.99) (end 91.44 50.8) (width 0.25) (layer F.Cu) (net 2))
 (segment (start 107.91 52.07) (end 107.91 49.49) (width 0.25) (layer F.Cu) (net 2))
 (segment (start 91.44 50.8) (end 91.44 55.88) (width 0.25) (layer F.Cu) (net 2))
 (segment (start 100.33 59.69) (end 103.505 59.69) (width 0.25) (layer F.Cu) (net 2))
 (segment (start 99.695 58.42) (end 100.33 59.055) (width 0.25) (layer F.Cu) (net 2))
 (segment (start 96.52 58.42) (end 99.695 58.42) (width 0.25) (layer F.Cu) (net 2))
 (segment (start 99.06 68.58) (end 96.52 68.58) (width 0.25) (layer F.Cu) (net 15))
 (segment (start 102.235 65.405) (end 99.06 68.58) (width 0.25) (layer F.Cu) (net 15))
 (segment (start 106.68 67.31) (end 104.775 65.405) (width 0.25) (layer F.Cu) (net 15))
 (segment (start 104.775 65.405) (end 102.235 65.405) (width 0.25) (layer F.Cu) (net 15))
 (segment (start 114.3 69.85) (end 111.76 67.31) (width 0.25) (layer F.Cu) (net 11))
 (segment (start 120.65 76.2) (end 114.3 69.85) (width 0.25) (layer F.Cu) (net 11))
 (segment (start 120.65 77.47) (end 120.65 76.2) (width 0.25) (layer F.Cu) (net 11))
 (segment (start 121.92 78.74) (end 120.65 77.47) (width 0.25) (layer F.Cu) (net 11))
 (segment (start 121.92 80.01) (end 121.92 78.74) (width 0.25) (layer F.Cu) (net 11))
 (segment (start 124.46 80.01) (end 124.46 78.74) (width 0.25) (layer F.Cu) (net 7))
 (segment (start 124.46 78.74) (end 125.73 77.47) (width 0.25) (layer F.Cu) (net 7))
 (segment (start 125.73 77.47) (end 125.73 72.39) (width 0.25) (layer F.Cu) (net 7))
 (segment (start 125.73 72.39) (end 123.19 69.85) (width 0.25) (layer F.Cu) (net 7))
 (segment (start 119.38 69.85) (end 116.84 67.31) (width 0.25) (layer F.Cu) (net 7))
 (segment (start 123.19 69.85) (end 119.38 69.85) (width 0.25) (layer F.Cu) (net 7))
 (segment (start 119.38 77.47) (end 119.38 80.01) (width 0.25) (layer F.Cu) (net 13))
 (segment (start 109.22 67.31) (end 119.38 77.47) (width 0.25) (layer F.Cu) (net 13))
 (segment (start 99.06 76.2) (end 96.52 76.2) (width 0.25) (layer F.Cu) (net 19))
 (segment (start 102.235 73.025) (end 99.06 76.2) (width 0.25) (layer F.Cu) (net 19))
 (segment (start 109.855 73.025) (end 102.235 73.025) (width 0.25) (layer F.Cu) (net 19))
 (segment (start 114.3 77.47) (end 109.855 73.025) (width 0.25) (layer F.Cu) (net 19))
 (segment (start 114.3 80.01) (end 114.3 77.47) (width 0.25) (layer F.Cu) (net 19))
 (segment (start 111.76 80.01) (end 111.76 76.835) (width 0.25) (layer F.Cu) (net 18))
 (segment (start 111.76 76.835) (end 109.22 74.295) (width 0.25) (layer F.Cu) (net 18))
 (segment (start 109.22 74.295) (end 102.87 74.295) (width 0.25) (layer F.Cu) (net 18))
 (segment (start 98.425 78.74) (end 96.52 78.74) (width 0.25) (layer F.Cu) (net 18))
 (segment (start 102.87 74.295) (end 98.425 78.74) (width 0.25) (layer F.Cu) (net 18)))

